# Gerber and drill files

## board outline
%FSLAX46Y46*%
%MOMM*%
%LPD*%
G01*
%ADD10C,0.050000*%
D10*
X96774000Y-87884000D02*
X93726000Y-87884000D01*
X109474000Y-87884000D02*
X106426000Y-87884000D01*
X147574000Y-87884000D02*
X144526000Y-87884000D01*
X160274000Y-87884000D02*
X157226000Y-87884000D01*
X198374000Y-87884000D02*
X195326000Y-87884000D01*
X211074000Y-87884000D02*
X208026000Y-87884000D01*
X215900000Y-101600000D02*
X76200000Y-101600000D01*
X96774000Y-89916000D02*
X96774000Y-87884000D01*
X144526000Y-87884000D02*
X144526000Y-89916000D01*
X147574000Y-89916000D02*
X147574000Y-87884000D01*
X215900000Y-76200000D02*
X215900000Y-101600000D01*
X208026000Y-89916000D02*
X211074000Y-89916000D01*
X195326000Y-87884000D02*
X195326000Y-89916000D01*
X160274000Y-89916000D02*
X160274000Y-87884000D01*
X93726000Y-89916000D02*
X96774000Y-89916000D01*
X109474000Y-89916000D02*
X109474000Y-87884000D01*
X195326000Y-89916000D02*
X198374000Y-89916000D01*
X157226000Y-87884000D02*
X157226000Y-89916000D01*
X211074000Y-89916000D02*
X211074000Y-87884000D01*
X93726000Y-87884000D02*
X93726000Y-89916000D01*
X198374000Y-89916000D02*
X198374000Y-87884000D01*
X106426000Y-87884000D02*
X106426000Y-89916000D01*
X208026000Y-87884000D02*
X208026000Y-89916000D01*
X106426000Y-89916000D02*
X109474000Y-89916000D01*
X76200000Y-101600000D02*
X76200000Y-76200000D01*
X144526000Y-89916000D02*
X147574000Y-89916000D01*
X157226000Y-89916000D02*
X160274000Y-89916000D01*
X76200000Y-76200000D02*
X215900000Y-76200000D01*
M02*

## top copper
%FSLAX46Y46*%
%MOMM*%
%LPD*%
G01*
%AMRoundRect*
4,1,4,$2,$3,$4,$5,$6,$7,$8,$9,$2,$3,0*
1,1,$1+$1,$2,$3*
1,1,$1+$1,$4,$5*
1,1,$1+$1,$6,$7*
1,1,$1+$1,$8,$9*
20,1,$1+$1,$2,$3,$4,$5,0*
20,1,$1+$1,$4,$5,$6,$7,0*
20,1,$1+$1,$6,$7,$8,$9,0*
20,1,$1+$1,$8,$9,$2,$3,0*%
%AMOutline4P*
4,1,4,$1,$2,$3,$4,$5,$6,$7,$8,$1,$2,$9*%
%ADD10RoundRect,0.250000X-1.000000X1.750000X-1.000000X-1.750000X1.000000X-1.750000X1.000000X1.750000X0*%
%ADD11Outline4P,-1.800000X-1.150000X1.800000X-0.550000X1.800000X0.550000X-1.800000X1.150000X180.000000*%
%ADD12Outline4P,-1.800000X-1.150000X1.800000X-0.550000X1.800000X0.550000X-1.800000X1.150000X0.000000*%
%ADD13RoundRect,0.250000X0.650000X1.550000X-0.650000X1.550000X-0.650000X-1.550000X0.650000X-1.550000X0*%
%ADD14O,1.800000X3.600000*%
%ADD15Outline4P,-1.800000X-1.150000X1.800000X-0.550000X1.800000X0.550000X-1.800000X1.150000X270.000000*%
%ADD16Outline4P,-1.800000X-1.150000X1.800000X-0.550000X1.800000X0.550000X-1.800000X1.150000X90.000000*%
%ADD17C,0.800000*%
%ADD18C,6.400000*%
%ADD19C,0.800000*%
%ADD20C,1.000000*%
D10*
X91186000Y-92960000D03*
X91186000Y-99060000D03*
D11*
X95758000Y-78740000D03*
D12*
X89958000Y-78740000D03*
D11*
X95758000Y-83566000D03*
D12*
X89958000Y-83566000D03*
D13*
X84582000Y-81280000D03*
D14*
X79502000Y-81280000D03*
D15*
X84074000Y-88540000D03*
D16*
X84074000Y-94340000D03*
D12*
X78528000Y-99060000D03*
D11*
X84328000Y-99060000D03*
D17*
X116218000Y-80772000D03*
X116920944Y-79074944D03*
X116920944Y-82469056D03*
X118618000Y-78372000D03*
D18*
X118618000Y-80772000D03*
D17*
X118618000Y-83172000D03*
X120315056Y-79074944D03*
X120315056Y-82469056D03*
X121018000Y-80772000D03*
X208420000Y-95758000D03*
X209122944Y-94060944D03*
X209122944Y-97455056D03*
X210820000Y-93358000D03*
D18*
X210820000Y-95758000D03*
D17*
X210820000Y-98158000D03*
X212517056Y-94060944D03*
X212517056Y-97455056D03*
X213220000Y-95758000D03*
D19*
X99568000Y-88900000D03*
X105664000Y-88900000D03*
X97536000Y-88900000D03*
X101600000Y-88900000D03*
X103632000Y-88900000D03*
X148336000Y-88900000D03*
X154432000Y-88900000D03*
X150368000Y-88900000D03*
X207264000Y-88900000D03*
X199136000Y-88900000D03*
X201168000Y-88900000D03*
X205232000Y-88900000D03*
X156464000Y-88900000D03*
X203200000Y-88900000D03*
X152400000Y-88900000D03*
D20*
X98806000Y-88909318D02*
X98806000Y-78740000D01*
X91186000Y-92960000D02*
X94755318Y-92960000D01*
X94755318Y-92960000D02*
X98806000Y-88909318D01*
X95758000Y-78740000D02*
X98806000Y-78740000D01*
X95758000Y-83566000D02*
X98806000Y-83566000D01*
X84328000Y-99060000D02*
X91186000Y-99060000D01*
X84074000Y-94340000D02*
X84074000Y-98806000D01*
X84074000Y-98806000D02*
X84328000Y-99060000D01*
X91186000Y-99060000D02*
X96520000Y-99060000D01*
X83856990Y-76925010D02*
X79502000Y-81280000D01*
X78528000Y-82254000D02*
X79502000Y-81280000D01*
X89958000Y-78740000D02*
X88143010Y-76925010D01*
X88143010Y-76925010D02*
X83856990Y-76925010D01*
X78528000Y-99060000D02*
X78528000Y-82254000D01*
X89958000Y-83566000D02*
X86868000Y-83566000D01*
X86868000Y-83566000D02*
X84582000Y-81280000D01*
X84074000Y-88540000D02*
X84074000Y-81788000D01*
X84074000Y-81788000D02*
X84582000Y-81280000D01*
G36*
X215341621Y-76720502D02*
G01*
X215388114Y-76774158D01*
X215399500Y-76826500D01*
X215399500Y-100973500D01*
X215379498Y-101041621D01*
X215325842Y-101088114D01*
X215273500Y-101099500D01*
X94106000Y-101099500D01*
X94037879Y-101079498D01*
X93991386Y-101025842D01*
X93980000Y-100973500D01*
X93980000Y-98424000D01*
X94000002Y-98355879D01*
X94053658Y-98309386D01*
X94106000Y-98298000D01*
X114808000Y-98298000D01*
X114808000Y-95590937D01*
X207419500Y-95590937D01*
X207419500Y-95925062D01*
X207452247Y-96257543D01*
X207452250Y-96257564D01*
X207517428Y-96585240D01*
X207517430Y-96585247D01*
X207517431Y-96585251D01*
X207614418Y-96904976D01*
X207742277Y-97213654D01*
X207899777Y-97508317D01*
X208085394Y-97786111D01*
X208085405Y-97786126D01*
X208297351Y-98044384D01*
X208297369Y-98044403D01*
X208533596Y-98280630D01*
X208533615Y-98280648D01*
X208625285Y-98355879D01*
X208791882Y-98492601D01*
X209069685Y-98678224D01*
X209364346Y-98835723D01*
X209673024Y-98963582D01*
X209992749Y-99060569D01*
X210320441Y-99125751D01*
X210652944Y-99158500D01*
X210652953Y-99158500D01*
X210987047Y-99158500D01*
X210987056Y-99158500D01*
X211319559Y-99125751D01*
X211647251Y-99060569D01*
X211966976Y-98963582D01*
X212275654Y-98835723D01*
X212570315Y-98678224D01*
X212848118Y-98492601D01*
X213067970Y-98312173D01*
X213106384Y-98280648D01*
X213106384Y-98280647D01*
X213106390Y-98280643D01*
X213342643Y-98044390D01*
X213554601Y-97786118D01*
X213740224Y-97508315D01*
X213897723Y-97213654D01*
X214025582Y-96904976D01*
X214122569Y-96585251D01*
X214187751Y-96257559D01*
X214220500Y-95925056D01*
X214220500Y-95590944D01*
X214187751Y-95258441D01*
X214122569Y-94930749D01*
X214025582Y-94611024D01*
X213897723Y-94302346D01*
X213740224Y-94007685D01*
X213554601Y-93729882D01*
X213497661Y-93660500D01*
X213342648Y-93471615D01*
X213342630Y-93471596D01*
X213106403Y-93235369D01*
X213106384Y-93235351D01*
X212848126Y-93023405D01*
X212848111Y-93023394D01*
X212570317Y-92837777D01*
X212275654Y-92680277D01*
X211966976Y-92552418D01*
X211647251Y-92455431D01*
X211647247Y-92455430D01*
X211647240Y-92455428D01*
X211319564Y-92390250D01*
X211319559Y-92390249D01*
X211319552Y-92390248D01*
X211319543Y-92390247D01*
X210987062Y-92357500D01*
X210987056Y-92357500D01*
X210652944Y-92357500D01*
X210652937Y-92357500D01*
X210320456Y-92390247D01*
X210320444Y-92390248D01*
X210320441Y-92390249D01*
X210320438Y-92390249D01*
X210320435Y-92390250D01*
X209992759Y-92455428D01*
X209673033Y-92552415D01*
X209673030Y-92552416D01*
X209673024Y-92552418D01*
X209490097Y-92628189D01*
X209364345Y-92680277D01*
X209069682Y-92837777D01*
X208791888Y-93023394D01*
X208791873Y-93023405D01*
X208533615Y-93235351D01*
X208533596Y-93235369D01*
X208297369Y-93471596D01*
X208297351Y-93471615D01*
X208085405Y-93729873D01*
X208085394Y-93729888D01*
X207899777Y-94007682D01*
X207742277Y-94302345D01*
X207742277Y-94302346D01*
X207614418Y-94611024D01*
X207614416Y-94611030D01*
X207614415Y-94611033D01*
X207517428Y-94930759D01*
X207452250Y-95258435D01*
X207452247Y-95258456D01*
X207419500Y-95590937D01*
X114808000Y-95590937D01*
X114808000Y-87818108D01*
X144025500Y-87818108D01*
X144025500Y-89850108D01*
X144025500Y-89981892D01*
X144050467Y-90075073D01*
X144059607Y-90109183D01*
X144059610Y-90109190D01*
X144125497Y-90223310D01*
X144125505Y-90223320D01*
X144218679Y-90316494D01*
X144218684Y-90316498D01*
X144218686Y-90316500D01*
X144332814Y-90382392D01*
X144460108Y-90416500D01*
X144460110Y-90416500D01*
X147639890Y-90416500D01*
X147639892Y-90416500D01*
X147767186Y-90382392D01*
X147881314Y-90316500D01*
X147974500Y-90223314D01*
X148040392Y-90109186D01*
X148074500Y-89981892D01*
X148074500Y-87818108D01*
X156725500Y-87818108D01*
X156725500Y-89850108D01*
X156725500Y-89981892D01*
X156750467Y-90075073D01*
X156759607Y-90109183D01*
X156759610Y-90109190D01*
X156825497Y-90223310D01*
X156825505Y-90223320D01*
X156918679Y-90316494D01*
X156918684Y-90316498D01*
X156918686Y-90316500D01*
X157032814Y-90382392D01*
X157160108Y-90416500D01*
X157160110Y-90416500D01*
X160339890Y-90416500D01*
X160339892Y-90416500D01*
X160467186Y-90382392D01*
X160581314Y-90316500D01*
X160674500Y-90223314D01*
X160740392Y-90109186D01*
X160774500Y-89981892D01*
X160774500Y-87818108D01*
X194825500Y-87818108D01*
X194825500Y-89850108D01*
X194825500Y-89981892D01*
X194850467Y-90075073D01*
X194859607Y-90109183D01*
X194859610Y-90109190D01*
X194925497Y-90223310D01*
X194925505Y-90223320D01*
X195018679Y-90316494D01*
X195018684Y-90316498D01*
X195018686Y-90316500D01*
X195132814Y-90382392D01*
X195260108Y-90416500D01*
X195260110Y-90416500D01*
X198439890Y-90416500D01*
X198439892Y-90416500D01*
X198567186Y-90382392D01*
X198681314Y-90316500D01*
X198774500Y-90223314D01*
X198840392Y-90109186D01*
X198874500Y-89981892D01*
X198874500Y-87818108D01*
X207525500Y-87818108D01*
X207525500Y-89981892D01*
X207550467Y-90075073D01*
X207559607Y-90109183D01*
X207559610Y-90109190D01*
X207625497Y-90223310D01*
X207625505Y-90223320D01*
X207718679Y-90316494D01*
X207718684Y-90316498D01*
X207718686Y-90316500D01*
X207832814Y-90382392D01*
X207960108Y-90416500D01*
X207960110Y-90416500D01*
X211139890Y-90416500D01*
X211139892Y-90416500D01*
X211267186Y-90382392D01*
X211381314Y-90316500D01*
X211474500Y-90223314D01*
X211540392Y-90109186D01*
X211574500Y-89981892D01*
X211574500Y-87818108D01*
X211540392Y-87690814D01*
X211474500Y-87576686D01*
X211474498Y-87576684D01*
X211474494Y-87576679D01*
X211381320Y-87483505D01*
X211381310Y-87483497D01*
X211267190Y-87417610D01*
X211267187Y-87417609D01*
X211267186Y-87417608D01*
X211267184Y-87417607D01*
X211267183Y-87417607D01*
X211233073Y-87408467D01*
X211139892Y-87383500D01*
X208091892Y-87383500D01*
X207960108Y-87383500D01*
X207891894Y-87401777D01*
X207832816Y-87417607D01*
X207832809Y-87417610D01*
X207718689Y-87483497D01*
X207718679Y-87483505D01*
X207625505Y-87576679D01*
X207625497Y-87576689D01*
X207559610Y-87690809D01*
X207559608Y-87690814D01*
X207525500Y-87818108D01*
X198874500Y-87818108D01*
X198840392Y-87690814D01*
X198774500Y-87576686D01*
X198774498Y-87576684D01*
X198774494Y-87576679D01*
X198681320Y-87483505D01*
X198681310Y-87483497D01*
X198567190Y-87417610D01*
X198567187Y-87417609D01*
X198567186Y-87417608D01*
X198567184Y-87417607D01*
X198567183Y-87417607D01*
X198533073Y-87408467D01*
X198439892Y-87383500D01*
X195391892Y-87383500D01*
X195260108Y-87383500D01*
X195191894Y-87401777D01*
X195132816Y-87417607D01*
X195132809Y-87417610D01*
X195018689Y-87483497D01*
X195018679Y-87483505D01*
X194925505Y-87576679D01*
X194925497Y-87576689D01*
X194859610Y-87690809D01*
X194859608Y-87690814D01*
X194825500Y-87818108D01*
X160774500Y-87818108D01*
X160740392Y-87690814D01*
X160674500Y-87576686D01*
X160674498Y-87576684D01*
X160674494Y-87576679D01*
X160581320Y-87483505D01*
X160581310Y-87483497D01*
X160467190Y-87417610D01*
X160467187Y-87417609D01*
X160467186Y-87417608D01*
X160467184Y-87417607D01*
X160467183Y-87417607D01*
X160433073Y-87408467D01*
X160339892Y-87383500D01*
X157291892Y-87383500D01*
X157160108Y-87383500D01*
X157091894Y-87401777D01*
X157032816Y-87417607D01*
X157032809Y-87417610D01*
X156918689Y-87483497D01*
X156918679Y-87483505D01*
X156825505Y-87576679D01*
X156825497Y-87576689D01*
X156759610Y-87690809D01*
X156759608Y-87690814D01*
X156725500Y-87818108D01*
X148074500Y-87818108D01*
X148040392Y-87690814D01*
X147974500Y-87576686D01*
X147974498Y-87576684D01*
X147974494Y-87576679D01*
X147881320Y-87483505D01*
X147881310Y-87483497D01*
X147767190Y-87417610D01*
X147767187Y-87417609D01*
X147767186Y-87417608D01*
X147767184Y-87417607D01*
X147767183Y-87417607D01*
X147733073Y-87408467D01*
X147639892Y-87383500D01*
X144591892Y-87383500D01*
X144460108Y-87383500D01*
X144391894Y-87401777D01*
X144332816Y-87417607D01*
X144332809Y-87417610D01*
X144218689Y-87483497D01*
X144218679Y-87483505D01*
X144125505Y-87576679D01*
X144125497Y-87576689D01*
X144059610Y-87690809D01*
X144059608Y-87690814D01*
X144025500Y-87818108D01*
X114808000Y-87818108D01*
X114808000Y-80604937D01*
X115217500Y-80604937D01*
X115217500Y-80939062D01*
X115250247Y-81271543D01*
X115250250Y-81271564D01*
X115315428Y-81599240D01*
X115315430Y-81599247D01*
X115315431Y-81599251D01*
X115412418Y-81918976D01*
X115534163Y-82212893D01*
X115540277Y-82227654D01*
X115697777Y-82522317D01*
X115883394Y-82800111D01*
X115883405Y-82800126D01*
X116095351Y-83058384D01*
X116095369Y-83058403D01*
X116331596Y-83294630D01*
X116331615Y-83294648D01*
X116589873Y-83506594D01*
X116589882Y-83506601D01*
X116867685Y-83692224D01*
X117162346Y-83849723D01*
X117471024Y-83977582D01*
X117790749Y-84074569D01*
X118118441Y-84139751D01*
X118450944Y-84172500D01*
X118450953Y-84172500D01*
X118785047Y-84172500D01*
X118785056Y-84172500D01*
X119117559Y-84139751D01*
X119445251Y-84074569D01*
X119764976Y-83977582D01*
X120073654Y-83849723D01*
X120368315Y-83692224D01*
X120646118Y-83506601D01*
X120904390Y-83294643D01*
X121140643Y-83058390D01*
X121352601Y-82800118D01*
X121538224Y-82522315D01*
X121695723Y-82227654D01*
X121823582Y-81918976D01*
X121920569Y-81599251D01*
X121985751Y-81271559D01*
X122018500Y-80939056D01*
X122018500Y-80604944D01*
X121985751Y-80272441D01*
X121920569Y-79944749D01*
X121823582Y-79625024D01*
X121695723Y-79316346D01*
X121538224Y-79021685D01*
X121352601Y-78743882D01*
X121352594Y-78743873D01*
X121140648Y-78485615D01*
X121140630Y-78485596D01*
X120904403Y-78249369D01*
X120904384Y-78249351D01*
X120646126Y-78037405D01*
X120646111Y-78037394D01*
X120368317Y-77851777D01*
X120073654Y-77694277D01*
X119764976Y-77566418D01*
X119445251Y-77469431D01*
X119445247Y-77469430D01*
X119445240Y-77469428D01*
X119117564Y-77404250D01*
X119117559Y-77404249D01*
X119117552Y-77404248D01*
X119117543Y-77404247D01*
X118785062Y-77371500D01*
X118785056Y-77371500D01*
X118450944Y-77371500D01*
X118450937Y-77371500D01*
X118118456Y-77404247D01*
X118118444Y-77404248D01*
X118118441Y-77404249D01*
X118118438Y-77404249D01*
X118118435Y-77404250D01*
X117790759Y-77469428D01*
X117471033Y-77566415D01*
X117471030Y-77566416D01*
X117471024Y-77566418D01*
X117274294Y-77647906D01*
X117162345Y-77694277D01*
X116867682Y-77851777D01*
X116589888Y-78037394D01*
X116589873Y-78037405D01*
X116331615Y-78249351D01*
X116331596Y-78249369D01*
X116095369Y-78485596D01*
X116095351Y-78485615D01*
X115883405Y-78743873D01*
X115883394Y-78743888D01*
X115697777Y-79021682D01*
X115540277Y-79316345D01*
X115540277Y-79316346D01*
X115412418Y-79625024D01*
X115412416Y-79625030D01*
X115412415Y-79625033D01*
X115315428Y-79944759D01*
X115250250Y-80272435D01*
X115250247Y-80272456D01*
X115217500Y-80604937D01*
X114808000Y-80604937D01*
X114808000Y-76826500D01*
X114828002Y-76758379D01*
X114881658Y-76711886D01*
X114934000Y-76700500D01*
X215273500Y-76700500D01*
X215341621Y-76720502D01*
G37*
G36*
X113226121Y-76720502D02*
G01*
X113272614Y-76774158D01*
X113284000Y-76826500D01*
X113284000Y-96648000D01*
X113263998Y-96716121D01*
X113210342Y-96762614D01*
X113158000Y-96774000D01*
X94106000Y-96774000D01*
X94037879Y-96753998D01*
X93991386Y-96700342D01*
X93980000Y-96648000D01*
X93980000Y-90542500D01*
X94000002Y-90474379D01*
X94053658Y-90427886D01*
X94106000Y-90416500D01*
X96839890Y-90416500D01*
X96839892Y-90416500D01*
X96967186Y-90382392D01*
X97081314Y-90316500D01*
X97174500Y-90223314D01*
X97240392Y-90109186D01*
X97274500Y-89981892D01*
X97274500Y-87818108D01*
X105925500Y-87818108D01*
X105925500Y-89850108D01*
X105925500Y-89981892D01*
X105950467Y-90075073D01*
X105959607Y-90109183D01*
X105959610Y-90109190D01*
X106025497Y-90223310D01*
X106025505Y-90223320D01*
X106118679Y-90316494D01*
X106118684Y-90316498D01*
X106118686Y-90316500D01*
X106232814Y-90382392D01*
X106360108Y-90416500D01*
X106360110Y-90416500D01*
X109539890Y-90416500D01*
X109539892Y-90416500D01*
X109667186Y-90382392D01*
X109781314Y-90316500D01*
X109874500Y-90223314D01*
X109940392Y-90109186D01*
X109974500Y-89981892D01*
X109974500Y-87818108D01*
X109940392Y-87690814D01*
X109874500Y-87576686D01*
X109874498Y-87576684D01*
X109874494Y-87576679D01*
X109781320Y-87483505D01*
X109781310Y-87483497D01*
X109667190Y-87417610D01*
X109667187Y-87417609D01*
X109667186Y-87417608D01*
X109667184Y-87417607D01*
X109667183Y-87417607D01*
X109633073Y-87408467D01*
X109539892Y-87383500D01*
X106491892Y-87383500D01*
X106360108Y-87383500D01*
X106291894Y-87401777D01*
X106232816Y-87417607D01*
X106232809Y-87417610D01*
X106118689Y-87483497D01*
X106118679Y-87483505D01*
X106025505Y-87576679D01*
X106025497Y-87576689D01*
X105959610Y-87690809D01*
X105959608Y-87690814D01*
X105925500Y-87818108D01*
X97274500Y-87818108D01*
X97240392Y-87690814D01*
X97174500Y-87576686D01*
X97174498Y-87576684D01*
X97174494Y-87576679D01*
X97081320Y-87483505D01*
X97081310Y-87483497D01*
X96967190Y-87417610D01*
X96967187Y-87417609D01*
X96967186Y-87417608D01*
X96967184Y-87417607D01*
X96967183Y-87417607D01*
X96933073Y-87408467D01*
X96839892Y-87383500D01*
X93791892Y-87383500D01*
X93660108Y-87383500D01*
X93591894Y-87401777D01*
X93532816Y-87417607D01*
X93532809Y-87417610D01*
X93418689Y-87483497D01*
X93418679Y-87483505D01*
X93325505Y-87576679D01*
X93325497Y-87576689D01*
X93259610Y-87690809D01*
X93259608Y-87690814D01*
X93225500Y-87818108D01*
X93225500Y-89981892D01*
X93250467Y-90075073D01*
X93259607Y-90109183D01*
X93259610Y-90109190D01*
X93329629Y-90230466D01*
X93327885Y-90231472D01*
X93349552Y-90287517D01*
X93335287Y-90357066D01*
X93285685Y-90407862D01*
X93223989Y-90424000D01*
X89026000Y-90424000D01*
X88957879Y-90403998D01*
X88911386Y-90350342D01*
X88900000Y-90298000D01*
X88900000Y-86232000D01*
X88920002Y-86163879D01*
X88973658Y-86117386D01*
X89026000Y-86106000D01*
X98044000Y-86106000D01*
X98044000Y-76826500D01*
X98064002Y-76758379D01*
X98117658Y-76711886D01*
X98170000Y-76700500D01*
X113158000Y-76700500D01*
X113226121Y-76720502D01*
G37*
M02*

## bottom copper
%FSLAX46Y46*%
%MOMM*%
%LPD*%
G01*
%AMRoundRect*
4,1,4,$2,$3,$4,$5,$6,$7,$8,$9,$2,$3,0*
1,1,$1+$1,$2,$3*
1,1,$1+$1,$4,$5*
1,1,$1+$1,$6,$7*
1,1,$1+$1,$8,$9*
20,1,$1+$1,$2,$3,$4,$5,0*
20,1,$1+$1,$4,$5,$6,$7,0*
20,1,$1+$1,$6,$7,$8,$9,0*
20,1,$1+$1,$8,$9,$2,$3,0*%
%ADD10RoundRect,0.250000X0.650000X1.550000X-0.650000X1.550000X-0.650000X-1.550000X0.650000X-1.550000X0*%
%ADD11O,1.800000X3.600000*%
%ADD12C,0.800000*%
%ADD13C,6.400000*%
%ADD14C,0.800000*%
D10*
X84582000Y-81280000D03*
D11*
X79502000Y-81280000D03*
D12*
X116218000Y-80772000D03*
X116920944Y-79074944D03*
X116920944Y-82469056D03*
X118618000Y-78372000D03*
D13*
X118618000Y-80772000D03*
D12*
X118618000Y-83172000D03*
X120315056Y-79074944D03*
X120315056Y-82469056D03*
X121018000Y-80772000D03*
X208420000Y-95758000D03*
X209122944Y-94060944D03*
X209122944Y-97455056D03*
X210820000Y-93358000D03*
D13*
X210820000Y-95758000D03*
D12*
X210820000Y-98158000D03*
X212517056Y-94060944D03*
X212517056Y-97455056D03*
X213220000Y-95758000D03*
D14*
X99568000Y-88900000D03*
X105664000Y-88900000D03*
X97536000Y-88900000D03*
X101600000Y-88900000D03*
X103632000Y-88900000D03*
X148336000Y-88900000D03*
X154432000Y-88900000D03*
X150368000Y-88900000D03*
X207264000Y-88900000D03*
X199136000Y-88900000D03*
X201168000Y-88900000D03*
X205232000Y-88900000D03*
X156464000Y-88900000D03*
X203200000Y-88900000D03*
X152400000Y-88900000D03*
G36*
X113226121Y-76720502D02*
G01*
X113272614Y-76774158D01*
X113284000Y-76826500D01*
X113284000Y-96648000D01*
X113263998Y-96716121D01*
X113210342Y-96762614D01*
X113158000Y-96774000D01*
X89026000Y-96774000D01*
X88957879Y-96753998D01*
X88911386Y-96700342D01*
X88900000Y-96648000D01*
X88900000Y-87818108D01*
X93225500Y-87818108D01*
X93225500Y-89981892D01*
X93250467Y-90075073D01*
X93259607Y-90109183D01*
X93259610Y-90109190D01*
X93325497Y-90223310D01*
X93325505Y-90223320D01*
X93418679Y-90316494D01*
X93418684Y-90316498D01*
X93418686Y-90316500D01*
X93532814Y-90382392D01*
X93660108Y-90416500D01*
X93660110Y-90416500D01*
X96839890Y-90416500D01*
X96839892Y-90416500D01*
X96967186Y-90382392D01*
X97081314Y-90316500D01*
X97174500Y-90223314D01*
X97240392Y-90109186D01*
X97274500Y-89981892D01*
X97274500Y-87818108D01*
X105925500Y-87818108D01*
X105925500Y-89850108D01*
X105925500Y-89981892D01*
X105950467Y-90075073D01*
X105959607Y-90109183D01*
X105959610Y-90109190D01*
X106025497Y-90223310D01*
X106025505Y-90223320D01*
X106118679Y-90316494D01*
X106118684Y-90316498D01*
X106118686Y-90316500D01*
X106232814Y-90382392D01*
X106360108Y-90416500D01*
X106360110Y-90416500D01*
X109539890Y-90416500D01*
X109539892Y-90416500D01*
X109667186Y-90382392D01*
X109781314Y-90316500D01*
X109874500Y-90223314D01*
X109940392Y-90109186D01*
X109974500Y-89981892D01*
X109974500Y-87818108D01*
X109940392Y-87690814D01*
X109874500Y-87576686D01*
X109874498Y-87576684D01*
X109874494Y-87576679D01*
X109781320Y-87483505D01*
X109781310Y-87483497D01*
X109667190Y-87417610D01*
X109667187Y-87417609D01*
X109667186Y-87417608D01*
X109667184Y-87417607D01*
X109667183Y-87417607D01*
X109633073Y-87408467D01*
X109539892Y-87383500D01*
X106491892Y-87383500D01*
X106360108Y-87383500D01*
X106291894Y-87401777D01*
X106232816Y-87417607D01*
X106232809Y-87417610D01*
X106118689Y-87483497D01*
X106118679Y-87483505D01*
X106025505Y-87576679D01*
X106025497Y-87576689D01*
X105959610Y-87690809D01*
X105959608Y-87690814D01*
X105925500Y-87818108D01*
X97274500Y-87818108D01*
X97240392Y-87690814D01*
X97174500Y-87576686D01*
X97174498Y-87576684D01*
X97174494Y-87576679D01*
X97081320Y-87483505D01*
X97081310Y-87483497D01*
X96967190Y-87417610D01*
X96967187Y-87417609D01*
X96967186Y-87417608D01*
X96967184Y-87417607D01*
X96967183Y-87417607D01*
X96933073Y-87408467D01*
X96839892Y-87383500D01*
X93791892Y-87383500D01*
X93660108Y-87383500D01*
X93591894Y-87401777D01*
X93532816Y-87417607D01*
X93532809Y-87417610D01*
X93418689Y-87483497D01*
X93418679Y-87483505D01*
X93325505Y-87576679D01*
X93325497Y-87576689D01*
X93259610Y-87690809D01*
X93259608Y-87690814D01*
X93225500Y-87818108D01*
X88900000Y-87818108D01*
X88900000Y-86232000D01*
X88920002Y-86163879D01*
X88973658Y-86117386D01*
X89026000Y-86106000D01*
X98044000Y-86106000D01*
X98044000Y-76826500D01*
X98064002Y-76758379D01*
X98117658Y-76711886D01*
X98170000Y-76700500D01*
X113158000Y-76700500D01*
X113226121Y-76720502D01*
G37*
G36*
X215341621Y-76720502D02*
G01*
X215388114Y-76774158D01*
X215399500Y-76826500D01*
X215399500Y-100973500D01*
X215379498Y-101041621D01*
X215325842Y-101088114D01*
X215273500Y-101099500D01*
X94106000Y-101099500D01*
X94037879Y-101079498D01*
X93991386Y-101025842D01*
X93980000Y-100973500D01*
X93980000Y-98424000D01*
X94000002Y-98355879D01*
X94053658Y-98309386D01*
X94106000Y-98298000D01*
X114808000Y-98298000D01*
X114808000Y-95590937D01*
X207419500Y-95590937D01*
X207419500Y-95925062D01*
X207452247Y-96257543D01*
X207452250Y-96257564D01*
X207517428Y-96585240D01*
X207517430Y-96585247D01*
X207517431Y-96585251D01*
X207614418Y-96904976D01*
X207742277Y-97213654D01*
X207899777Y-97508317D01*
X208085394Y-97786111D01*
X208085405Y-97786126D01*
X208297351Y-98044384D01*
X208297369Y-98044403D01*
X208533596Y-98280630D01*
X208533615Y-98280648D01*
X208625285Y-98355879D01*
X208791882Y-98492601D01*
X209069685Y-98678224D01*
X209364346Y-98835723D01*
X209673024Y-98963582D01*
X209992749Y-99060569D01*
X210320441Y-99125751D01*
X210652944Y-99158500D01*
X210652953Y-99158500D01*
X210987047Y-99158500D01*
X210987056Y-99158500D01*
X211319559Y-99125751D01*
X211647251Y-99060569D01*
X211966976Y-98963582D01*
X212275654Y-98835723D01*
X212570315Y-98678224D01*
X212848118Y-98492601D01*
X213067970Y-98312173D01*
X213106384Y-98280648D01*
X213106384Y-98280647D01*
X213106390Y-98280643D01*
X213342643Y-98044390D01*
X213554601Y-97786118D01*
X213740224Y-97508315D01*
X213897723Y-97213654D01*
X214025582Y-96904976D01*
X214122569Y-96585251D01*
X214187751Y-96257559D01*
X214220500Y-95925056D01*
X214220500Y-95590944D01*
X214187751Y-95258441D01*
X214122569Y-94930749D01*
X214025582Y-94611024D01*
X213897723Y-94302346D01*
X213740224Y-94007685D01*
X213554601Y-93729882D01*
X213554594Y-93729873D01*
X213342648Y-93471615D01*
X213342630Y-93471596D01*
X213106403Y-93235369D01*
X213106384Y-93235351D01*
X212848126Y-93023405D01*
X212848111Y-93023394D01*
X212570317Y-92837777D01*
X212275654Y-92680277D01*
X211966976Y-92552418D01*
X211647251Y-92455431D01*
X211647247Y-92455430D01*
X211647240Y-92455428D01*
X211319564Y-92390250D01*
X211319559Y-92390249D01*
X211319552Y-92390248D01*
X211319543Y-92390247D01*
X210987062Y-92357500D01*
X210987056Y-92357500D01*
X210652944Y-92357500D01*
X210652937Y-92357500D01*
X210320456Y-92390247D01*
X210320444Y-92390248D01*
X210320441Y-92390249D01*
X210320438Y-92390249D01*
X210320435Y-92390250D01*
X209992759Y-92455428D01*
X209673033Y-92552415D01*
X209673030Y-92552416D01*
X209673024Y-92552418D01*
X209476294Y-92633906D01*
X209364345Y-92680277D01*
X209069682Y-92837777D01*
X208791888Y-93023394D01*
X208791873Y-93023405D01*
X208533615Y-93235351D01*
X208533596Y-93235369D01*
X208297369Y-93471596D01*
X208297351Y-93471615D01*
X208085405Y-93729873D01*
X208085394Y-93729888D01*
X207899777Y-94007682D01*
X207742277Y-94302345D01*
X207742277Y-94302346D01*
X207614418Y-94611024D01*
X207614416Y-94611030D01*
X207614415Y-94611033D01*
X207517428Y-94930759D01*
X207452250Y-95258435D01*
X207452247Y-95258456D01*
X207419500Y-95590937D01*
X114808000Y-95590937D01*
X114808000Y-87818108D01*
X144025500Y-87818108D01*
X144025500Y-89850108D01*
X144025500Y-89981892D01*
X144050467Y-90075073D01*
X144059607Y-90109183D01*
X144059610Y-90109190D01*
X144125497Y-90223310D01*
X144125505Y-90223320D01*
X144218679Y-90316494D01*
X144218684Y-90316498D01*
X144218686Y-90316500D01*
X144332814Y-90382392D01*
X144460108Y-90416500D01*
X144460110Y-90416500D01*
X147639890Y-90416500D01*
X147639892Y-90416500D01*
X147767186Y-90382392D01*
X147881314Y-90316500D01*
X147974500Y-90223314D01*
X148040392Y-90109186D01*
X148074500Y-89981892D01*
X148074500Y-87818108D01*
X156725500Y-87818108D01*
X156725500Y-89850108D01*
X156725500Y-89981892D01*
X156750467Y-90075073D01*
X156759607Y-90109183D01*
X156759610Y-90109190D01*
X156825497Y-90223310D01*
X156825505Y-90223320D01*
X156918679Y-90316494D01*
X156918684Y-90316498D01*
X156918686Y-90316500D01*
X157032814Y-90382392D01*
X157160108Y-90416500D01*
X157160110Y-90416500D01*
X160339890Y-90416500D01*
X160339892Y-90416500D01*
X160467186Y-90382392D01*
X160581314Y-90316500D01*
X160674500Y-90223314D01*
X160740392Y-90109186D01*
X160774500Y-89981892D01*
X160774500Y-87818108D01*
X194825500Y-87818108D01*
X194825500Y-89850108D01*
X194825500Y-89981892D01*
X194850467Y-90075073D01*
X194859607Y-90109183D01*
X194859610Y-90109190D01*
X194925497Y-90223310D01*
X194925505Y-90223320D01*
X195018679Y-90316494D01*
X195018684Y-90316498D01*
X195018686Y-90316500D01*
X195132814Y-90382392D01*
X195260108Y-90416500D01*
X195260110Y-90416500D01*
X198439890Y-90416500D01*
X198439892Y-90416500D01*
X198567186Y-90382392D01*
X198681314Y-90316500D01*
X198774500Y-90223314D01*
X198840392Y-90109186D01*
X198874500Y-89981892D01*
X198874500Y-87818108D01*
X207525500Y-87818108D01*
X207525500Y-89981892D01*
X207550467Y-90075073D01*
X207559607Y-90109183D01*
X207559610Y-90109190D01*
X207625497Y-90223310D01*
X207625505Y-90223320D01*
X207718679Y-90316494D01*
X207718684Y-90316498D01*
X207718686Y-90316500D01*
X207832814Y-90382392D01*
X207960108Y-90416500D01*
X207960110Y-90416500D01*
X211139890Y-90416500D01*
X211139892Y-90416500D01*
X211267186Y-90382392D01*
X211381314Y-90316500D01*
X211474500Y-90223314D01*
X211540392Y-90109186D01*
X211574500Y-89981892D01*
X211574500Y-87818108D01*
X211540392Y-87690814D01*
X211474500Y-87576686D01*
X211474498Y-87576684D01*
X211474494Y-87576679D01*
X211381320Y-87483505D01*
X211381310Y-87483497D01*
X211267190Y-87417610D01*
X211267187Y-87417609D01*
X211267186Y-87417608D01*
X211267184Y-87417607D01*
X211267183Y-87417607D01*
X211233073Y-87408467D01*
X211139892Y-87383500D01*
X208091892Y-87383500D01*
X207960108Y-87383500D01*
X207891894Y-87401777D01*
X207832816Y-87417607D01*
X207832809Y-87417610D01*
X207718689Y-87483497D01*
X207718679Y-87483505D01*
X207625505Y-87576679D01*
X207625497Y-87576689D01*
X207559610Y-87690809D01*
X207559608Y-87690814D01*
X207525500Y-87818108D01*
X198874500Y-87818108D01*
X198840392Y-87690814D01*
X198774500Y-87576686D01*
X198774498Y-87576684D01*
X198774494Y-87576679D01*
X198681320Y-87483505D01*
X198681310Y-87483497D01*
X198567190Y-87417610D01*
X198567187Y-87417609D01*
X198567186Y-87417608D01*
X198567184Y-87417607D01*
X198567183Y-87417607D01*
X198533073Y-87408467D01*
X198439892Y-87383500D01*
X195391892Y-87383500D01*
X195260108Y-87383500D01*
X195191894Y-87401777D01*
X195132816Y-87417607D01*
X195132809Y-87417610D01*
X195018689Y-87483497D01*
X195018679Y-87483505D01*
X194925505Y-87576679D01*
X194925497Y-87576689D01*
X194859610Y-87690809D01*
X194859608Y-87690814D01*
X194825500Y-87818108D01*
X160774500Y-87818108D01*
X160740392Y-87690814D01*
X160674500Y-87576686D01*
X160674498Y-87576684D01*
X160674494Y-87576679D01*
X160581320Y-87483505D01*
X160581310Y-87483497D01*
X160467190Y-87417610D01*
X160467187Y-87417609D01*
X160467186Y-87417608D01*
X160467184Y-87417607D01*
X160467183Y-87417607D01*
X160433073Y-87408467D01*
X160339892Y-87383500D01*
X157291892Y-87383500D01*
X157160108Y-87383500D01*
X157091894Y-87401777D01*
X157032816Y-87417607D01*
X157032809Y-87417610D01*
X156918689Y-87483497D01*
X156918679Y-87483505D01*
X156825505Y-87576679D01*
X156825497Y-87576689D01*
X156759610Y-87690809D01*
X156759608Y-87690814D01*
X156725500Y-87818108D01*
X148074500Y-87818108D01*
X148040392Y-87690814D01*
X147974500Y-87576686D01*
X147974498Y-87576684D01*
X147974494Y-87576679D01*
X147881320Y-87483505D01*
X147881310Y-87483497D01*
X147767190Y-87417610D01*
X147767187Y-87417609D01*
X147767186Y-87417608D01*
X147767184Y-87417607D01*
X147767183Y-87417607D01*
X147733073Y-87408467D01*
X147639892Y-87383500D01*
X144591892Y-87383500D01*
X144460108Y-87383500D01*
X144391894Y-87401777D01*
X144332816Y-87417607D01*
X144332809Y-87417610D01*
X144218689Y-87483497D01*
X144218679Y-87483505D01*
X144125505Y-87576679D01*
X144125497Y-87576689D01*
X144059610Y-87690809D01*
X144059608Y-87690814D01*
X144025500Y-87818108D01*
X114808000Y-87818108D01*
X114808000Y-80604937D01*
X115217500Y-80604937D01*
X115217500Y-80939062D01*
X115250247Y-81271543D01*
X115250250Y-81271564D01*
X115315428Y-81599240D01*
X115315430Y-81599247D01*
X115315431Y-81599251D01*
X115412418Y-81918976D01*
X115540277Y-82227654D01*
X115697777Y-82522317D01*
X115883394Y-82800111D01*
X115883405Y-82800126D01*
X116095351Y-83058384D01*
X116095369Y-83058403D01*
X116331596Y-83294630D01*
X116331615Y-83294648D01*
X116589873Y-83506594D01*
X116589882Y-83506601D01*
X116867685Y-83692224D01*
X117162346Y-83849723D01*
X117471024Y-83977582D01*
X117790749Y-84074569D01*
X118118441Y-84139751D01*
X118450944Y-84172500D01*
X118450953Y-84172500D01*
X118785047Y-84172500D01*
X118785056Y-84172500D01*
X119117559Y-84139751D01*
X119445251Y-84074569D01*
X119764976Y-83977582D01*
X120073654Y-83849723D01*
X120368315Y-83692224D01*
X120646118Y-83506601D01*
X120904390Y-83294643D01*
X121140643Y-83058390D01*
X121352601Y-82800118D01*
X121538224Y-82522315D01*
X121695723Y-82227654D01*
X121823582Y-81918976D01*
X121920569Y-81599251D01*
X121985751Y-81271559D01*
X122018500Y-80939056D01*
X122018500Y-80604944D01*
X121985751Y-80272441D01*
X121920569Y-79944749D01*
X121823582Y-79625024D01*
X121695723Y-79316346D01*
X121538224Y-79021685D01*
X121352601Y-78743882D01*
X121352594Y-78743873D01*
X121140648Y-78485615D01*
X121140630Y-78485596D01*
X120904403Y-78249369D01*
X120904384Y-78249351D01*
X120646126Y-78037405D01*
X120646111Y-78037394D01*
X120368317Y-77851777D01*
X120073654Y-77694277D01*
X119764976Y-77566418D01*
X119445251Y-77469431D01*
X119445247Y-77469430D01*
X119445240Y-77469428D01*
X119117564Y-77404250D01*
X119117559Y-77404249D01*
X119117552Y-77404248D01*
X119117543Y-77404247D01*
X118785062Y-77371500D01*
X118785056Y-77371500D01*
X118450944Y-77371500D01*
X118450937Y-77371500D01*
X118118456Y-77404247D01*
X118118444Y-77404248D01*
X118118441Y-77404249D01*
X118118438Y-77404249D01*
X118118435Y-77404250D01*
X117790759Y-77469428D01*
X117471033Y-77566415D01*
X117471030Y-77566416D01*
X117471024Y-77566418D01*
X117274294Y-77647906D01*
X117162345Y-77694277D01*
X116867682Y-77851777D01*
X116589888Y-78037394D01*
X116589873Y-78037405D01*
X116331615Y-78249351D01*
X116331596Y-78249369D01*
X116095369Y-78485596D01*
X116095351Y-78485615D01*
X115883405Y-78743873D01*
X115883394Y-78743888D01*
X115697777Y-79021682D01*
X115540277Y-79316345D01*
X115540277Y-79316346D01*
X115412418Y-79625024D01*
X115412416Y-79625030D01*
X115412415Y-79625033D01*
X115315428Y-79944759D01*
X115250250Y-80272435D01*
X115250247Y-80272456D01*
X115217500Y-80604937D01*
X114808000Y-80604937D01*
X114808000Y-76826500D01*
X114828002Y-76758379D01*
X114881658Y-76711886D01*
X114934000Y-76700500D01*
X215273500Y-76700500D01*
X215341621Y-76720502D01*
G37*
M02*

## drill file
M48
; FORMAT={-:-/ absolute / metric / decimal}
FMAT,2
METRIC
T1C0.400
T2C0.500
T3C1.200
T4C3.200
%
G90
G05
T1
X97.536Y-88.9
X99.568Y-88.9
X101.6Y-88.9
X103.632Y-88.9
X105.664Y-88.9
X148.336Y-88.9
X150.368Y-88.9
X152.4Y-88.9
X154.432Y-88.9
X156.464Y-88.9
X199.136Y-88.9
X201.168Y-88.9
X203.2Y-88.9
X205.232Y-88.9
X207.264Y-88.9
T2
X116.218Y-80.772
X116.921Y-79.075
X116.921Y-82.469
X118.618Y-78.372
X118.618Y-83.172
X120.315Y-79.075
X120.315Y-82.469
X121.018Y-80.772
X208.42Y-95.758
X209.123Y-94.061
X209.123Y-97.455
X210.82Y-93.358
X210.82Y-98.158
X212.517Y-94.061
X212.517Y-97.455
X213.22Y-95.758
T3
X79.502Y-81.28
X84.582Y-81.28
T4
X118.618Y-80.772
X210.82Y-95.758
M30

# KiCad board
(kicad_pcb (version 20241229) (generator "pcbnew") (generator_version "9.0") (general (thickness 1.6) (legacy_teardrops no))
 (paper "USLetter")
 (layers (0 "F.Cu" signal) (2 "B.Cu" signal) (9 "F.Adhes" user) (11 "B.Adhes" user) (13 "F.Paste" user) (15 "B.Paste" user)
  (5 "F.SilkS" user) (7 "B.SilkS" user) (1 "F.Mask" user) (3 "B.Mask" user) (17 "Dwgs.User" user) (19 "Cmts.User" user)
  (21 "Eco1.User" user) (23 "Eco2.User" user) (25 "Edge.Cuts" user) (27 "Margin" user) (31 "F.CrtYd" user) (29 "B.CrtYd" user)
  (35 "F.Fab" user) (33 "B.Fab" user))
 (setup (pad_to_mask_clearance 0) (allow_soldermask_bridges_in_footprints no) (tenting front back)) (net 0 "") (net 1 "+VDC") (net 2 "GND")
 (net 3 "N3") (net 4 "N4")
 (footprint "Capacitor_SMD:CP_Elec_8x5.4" (layer "F.Cu") (at 91.186 96.01 -90)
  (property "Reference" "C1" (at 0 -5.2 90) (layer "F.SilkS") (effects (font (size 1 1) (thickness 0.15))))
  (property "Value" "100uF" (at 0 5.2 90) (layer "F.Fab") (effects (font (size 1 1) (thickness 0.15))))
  (pad "1" smd roundrect (at -3.05 0 270) (size 4 2.5) (layers "F.Cu" "F.Mask" "F.Paste") (roundrect_rratio 0.1) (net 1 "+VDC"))
  (pad "2" smd roundrect (at 3.05 0 270) (size 4 2.5) (layers "F.Cu" "F.Mask" "F.Paste") (roundrect_rratio 0.1) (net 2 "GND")))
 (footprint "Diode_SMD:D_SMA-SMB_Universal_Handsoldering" (layer "F.Cu") (at 92.858 78.74 180)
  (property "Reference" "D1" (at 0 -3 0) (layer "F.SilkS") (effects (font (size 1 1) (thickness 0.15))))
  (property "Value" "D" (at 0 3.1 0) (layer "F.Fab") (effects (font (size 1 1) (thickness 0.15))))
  (pad "1" smd trapezoid (at -2.9 0 180) (size 3.6 1.7) (rect_delta 0.6 0) (layers "F.Cu" "F.Mask" "F.Paste") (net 1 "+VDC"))
  (pad "2" smd trapezoid (at 2.9 0) (size 3.6 1.7) (rect_delta 0.6 0) (layers "F.Cu" "F.Mask" "F.Paste") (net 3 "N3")))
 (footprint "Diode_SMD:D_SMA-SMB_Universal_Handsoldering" (layer "F.Cu") (at 92.858 83.566 180)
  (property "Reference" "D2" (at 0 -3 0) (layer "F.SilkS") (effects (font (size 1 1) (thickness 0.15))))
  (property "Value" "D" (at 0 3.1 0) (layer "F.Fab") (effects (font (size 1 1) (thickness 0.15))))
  (pad "1" smd trapezoid (at -2.9 0 180) (size 3.6 1.7) (rect_delta 0.6 0) (layers "F.Cu" "F.Mask" "F.Paste") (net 1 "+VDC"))
  (pad "2" smd trapezoid (at 2.9 0) (size 3.6 1.7) (rect_delta 0.6 0) (layers "F.Cu" "F.Mask" "F.Paste") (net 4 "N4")))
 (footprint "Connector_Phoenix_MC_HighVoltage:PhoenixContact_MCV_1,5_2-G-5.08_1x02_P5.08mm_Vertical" (layer "F.Cu") (at 84.582 81.28 180)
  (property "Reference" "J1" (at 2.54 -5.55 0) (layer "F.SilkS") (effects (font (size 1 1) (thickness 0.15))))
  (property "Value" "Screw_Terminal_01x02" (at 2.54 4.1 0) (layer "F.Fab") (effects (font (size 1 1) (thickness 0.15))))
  (pad "1" thru_hole roundrect (at 0 0 180) (size 1.8 3.6) (drill 1.2) (layers "*.Cu" "*.Mask") (remove_unused_layers no)
   (roundrect_rratio 0.1388888889) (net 4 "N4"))
  (pad "2" thru_hole oval (at 5.08 0 180) (size 1.8 3.6) (drill 1.2) (layers "*.Cu" "*.Mask") (remove_unused_layers no) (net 3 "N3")))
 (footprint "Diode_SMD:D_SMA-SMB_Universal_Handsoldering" (layer "F.Cu") (at 84.074 91.44 -90)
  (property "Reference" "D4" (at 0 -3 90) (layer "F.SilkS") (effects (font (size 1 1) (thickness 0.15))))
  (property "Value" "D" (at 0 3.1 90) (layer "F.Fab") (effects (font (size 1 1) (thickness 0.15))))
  (pad "1" smd trapezoid (at -2.9 0 270) (size 3.6 1.7) (rect_delta 0.6 0) (layers "F.Cu" "F.Mask" "F.Paste") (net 4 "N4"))
  (pad "2" smd trapezoid (at 2.9 0 90) (size 3.6 1.7) (rect_delta 0.6 0) (layers "F.Cu" "F.Mask" "F.Paste") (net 2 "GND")))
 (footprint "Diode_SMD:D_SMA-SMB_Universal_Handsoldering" (layer "F.Cu") (at 81.428 99.06)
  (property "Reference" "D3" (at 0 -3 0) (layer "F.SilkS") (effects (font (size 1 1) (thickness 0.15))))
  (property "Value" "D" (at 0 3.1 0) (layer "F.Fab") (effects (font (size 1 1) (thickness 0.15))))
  (pad "1" smd trapezoid (at -2.9 0) (size 3.6 1.7) (rect_delta 0.6 0) (layers "F.Cu" "F.Mask" "F.Paste") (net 3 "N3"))
  (pad "2" smd trapezoid (at 2.9 0 180) (size 3.6 1.7) (rect_delta 0.6 0) (layers "F.Cu" "F.Mask" "F.Paste") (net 2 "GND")))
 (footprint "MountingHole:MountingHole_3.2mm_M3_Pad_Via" (layer "F.Cu") (at 118.618 80.772)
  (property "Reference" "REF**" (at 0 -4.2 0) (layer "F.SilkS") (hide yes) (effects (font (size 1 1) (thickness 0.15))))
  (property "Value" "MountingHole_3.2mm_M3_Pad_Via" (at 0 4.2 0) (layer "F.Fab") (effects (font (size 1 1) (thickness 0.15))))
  (pad "1" thru_hole circle (at -2.4 0) (size 0.8 0.8) (drill 0.5) (layers "*.Cu" "*.Mask") (remove_unused_layers no))
  (pad "1" thru_hole circle (at -1.697056 -1.697056) (size 0.8 0.8) (drill 0.5) (layers "*.Cu" "*.Mask") (remove_unused_layers no))
  (pad "1" thru_hole circle (at -1.697056 1.697056) (size 0.8 0.8) (drill 0.5) (layers "*.Cu" "*.Mask") (remove_unused_layers no))
  (pad "1" thru_hole circle (at 0 -2.4) (size 0.8 0.8) (drill 0.5) (layers "*.Cu" "*.Mask") (remove_unused_layers no))
  (pad "1" thru_hole circle (at 0 0) (size 6.4 6.4) (drill 3.2) (layers "*.Cu" "*.Mask") (remove_unused_layers no))
  (pad "1" thru_hole circle (at 0 2.4) (size 0.8 0.8) (drill 0.5) (layers "*.Cu" "*.Mask") (remove_unused_layers no))
  (pad "1" thru_hole circle (at 1.697056 -1.697056) (size 0.8 0.8) (drill 0.5) (layers "*.Cu" "*.Mask") (remove_unused_layers no))
  (pad "1" thru_hole circle (at 1.697056 1.697056) (size 0.8 0.8) (drill 0.5) (layers "*.Cu" "*.Mask") (remove_unused_layers no))
  (pad "1" thru_hole circle (at 2.4 0) (size 0.8 0.8) (drill 0.5) (layers "*.Cu" "*.Mask") (remove_unused_layers no)))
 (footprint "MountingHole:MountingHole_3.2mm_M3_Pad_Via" (layer "F.Cu") (at 210.82 95.758)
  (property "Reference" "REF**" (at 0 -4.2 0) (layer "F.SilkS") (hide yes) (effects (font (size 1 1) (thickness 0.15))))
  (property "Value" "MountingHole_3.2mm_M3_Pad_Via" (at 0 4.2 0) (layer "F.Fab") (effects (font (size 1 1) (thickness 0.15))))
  (pad "1" thru_hole circle (at -2.4 0) (size 0.8 0.8) (drill 0.5) (layers "*.Cu" "*.Mask") (remove_unused_layers no))
  (pad "1" thru_hole circle (at -1.697056 -1.697056) (size 0.8 0.8) (drill 0.5) (layers "*.Cu" "*.Mask") (remove_unused_layers no))
  (pad "1" thru_hole circle (at -1.697056 1.697056) (size 0.8 0.8) (drill 0.5) (layers "*.Cu" "*.Mask") (remove_unused_layers no))
  (pad "1" thru_hole circle (at 0 -2.4) (size 0.8 0.8) (drill 0.5) (layers "*.Cu" "*.Mask") (remove_unused_layers no))
  (pad "1" thru_hole circle (at 0 0) (size 6.4 6.4) (drill 3.2) (layers "*.Cu" "*.Mask") (remove_unused_layers no))
  (pad "1" thru_hole circle (at 0 2.4) (size 0.8 0.8) (drill 0.5) (layers "*.Cu" "*.Mask") (remove_unused_layers no))
  (pad "1" thru_hole circle (at 1.697056 -1.697056) (size 0.8 0.8) (drill 0.5) (layers "*.Cu" "*.Mask") (remove_unused_layers no))
  (pad "1" thru_hole circle (at 1.697056 1.697056) (size 0.8 0.8) (drill 0.5) (layers "*.Cu" "*.Mask") (remove_unused_layers no))
  (pad "1" thru_hole circle (at 2.4 0) (size 0.8 0.8) (drill 0.5) (layers "*.Cu" "*.Mask") (remove_unused_layers no)))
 (gr_line (start 96.774 87.884) (end 93.726 87.884) (stroke (width 0.05) (type solid)) (layer "Edge.Cuts"))
 (gr_line (start 109.474 87.884) (end 106.426 87.884) (stroke (width 0.05) (type solid)) (layer "Edge.Cuts"))
 (gr_line (start 147.574 87.884) (end 144.526 87.884) (stroke (width 0.05) (type solid)) (layer "Edge.Cuts"))
 (gr_line (start 160.274 87.884) (end 157.226 87.884) (stroke (width 0.05) (type solid)) (layer "Edge.Cuts"))
 (gr_line (start 198.374 87.884) (end 195.326 87.884) (stroke (width 0.05) (type solid)) (layer "Edge.Cuts"))
 (gr_line (start 211.074 87.884) (end 208.026 87.884) (stroke (width 0.05) (type solid)) (layer "Edge.Cuts"))
 (gr_line (start 215.9 101.6) (end 76.2 101.6) (stroke (width 0.05) (type solid)) (layer "Edge.Cuts"))
 (gr_line (start 96.774 89.916) (end 96.774 87.884) (stroke (width 0.05) (type solid)) (layer "Edge.Cuts"))
 (gr_line (start 144.526 87.884) (end 144.526 89.916) (stroke (width 0.05) (type solid)) (layer "Edge.Cuts"))
 (gr_line (start 147.574 89.916) (end 147.574 87.884) (stroke (width 0.05) (type solid)) (layer "Edge.Cuts"))
 (gr_line (start 215.9 76.2) (end 215.9 101.6) (stroke (width 0.05) (type solid)) (layer "Edge.Cuts"))
 (gr_line (start 208.026 89.916) (end 211.074 89.916) (stroke (width 0.05) (type solid)) (layer "Edge.Cuts"))
 (gr_line (start 195.326 87.884) (end 195.326 89.916) (stroke (width 0.05) (type solid)) (layer "Edge.Cuts"))
 (gr_line (start 160.274 89.916) (end 160.274 87.884) (stroke (width 0.05) (type solid)) (layer "Edge.Cuts"))
 (gr_line (start 93.726 89.916) (end 96.774 89.916) (stroke (width 0.05) (type solid)) (layer "Edge.Cuts"))
 (gr_line (start 109.474 89.916) (end 109.474 87.884) (stroke (width 0.05) (type solid)) (layer "Edge.Cuts"))
 (gr_line (start 195.326 89.916) (end 198.374 89.916) (stroke (width 0.05) (type solid)) (layer "Edge.Cuts"))
 (gr_line (start 157.226 87.884) (end 157.226 89.916) (stroke (width 0.05) (type solid)) (layer "Edge.Cuts"))
 (gr_line (start 211.074 89.916) (end 211.074 87.884) (stroke (width 0.05) (type solid)) (layer "Edge.Cuts"))
 (gr_line (start 93.726 87.884) (end 93.726 89.916) (stroke (width 0.05) (type solid)) (layer "Edge.Cuts"))
 (gr_line (start 198.374 89.916) (end 198.374 87.884) (stroke (width 0.05) (type solid)) (layer "Edge.Cuts"))
 (gr_line (start 106.426 87.884) (end 106.426 89.916) (stroke (width 0.05) (type solid)) (layer "Edge.Cuts"))
 (gr_line (start 208.026 87.884) (end 208.026 89.916) (stroke (width 0.05) (type solid)) (layer "Edge.Cuts"))
 (gr_line (start 106.426 89.916) (end 109.474 89.916) (stroke (width 0.05) (type solid)) (layer "Edge.Cuts"))
 (gr_line (start 76.2 101.6) (end 76.2 76.2) (stroke (width 0.05) (type solid)) (layer "Edge.Cuts"))
 (gr_line (start 144.526 89.916) (end 147.574 89.916) (stroke (width 0.05) (type solid)) (layer "Edge.Cuts"))
 (gr_line (start 157.226 89.916) (end 160.274 89.916) (stroke (width 0.05) (type solid)) (layer "Edge.Cuts"))
 (gr_line (start 76.2 76.2) (end 215.9 76.2) (stroke (width 0.05) (type solid)) (layer "Edge.Cuts"))
 (segment (start 98.806 88.909318) (end 98.806 78.74) (width 1) (layer "F.Cu") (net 1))
 (segment (start 91.186 92.96) (end 94.755318 92.96) (width 1) (layer "F.Cu") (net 1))
 (segment (start 94.755318 92.96) (end 98.806 88.909318) (width 1) (layer "F.Cu") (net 1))
 (segment (start 95.758 78.74) (end 98.806 78.74) (width 1) (layer "F.Cu") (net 1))
 (segment (start 95.758 83.566) (end 98.806 83.566) (width 1) (layer "F.Cu") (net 1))
 (via (at 99.568 88.9) (size 0.8) (drill 0.4) (layers "F.Cu" "B.Cu") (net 1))
 (via (at 105.664 88.9) (size 0.8) (drill 0.4) (layers "F.Cu" "B.Cu") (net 1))
 (via (at 97.536 88.9) (size 0.8) (drill 0.4) (layers "F.Cu" "B.Cu") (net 1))
 (via (at 101.6 88.9) (size 0.8) (drill 0.4) (layers "F.Cu" "B.Cu") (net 1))
 (via (at 103.632 88.9) (size 0.8) (drill 0.4) (layers "F.Cu" "B.Cu") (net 1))
 (segment (start 84.328 99.06) (end 91.186 99.06) (width 1) (layer "F.Cu") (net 2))
 (segment (start 84.074 94.34) (end 84.074 98.806) (width 1) (layer "F.Cu") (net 2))
 (segment (start 84.074 98.806) (end 84.328 99.06) (width 1) (layer "F.Cu") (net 2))
 (segment (start 91.186 99.06) (end 96.52 99.06) (width 1) (layer "F.Cu") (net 2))
 (via (at 148.336 88.9) (size 0.8) (drill 0.4) (layers "F.Cu" "B.Cu") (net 2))
 (via (at 154.432 88.9) (size 0.8) (drill 0.4) (layers "F.Cu" "B.Cu") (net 2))
 (via (at 150.368 88.9) (size 0.8) (drill 0.4) (layers "F.Cu" "B.Cu") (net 2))
 (via (at 207.264 88.9) (size 0.8) (drill 0.4) (layers "F.Cu" "B.Cu") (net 2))
 (via (at 199.136 88.9) (size 0.8) (drill 0.4) (layers "F.Cu" "B.Cu") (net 2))
 (via (at 201.168 88.9) (size 0.8) (drill 0.4) (layers "F.Cu" "B.Cu") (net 2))
 (via (at 205.232 88.9) (size 0.8) (drill 0.4) (layers "F.Cu" "B.Cu") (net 2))
 (via (at 156.464 88.9) (size 0.8) (drill 0.4) (layers "F.Cu" "B.Cu") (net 2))
 (via (at 203.2 88.9) (size 0.8) (drill 0.4) (layers "F.Cu" "B.Cu") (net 2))
 (via (at 152.4 88.9) (size 0.8) (drill 0.4) (layers "F.Cu" "B.Cu") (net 2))
 (segment (start 83.85699 76.92501) (end 79.502 81.28) (width 1) (layer "F.Cu") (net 3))
 (segment (start 78.528 82.254) (end 79.502 81.28) (width 1) (layer "F.Cu") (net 3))
 (segment (start 89.958 78.74) (end 88.14301 76.92501) (width 1) (layer "F.Cu") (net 3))
 (segment (start 88.14301 76.92501) (end 83.85699 76.92501) (width 1) (layer "F.Cu") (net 3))
 (segment (start 78.528 99.06) (end 78.528 82.254) (width 1) (layer "F.Cu") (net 3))
 (segment (start 89.958 83.566) (end 86.868 83.566) (width 1) (layer "F.Cu") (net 4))
 (segment (start 86.868 83.566) (end 84.582 81.28) (width 1) (layer "F.Cu") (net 4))
 (segment (start 84.074 88.54) (end 84.074 81.788) (width 1) (layer "F.Cu") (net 4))
 (segment (start 84.074 81.788) (end 84.582 81.28) (width 1) (layer "F.Cu") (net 4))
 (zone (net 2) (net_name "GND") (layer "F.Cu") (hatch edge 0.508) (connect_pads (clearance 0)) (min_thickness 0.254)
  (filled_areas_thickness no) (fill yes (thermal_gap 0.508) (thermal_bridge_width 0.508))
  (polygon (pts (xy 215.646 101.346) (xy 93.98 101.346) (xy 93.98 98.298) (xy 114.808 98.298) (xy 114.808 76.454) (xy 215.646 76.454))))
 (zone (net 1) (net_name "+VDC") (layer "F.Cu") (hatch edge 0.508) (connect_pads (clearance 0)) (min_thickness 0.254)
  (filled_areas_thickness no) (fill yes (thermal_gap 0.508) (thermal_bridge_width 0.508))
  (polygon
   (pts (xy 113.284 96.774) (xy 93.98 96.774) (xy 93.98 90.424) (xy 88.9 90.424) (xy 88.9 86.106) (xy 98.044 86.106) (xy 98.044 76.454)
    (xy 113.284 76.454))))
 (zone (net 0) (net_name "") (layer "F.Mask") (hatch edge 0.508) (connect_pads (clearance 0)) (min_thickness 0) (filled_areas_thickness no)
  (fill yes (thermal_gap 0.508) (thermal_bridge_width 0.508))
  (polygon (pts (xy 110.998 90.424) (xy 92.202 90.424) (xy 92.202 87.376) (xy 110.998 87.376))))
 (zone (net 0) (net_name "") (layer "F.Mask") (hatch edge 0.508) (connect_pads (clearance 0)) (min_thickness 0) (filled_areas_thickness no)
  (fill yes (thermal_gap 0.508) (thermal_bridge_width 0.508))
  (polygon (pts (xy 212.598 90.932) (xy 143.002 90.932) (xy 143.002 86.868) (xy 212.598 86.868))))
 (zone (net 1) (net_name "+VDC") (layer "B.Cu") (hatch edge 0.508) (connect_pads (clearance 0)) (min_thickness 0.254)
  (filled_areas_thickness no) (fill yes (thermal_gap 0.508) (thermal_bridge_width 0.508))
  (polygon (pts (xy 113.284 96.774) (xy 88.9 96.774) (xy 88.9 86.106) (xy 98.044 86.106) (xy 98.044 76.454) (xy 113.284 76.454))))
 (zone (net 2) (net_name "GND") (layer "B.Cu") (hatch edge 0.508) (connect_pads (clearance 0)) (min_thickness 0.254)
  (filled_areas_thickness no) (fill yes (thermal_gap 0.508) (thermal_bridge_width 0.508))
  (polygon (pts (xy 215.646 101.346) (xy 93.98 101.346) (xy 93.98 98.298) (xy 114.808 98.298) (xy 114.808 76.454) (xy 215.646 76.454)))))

